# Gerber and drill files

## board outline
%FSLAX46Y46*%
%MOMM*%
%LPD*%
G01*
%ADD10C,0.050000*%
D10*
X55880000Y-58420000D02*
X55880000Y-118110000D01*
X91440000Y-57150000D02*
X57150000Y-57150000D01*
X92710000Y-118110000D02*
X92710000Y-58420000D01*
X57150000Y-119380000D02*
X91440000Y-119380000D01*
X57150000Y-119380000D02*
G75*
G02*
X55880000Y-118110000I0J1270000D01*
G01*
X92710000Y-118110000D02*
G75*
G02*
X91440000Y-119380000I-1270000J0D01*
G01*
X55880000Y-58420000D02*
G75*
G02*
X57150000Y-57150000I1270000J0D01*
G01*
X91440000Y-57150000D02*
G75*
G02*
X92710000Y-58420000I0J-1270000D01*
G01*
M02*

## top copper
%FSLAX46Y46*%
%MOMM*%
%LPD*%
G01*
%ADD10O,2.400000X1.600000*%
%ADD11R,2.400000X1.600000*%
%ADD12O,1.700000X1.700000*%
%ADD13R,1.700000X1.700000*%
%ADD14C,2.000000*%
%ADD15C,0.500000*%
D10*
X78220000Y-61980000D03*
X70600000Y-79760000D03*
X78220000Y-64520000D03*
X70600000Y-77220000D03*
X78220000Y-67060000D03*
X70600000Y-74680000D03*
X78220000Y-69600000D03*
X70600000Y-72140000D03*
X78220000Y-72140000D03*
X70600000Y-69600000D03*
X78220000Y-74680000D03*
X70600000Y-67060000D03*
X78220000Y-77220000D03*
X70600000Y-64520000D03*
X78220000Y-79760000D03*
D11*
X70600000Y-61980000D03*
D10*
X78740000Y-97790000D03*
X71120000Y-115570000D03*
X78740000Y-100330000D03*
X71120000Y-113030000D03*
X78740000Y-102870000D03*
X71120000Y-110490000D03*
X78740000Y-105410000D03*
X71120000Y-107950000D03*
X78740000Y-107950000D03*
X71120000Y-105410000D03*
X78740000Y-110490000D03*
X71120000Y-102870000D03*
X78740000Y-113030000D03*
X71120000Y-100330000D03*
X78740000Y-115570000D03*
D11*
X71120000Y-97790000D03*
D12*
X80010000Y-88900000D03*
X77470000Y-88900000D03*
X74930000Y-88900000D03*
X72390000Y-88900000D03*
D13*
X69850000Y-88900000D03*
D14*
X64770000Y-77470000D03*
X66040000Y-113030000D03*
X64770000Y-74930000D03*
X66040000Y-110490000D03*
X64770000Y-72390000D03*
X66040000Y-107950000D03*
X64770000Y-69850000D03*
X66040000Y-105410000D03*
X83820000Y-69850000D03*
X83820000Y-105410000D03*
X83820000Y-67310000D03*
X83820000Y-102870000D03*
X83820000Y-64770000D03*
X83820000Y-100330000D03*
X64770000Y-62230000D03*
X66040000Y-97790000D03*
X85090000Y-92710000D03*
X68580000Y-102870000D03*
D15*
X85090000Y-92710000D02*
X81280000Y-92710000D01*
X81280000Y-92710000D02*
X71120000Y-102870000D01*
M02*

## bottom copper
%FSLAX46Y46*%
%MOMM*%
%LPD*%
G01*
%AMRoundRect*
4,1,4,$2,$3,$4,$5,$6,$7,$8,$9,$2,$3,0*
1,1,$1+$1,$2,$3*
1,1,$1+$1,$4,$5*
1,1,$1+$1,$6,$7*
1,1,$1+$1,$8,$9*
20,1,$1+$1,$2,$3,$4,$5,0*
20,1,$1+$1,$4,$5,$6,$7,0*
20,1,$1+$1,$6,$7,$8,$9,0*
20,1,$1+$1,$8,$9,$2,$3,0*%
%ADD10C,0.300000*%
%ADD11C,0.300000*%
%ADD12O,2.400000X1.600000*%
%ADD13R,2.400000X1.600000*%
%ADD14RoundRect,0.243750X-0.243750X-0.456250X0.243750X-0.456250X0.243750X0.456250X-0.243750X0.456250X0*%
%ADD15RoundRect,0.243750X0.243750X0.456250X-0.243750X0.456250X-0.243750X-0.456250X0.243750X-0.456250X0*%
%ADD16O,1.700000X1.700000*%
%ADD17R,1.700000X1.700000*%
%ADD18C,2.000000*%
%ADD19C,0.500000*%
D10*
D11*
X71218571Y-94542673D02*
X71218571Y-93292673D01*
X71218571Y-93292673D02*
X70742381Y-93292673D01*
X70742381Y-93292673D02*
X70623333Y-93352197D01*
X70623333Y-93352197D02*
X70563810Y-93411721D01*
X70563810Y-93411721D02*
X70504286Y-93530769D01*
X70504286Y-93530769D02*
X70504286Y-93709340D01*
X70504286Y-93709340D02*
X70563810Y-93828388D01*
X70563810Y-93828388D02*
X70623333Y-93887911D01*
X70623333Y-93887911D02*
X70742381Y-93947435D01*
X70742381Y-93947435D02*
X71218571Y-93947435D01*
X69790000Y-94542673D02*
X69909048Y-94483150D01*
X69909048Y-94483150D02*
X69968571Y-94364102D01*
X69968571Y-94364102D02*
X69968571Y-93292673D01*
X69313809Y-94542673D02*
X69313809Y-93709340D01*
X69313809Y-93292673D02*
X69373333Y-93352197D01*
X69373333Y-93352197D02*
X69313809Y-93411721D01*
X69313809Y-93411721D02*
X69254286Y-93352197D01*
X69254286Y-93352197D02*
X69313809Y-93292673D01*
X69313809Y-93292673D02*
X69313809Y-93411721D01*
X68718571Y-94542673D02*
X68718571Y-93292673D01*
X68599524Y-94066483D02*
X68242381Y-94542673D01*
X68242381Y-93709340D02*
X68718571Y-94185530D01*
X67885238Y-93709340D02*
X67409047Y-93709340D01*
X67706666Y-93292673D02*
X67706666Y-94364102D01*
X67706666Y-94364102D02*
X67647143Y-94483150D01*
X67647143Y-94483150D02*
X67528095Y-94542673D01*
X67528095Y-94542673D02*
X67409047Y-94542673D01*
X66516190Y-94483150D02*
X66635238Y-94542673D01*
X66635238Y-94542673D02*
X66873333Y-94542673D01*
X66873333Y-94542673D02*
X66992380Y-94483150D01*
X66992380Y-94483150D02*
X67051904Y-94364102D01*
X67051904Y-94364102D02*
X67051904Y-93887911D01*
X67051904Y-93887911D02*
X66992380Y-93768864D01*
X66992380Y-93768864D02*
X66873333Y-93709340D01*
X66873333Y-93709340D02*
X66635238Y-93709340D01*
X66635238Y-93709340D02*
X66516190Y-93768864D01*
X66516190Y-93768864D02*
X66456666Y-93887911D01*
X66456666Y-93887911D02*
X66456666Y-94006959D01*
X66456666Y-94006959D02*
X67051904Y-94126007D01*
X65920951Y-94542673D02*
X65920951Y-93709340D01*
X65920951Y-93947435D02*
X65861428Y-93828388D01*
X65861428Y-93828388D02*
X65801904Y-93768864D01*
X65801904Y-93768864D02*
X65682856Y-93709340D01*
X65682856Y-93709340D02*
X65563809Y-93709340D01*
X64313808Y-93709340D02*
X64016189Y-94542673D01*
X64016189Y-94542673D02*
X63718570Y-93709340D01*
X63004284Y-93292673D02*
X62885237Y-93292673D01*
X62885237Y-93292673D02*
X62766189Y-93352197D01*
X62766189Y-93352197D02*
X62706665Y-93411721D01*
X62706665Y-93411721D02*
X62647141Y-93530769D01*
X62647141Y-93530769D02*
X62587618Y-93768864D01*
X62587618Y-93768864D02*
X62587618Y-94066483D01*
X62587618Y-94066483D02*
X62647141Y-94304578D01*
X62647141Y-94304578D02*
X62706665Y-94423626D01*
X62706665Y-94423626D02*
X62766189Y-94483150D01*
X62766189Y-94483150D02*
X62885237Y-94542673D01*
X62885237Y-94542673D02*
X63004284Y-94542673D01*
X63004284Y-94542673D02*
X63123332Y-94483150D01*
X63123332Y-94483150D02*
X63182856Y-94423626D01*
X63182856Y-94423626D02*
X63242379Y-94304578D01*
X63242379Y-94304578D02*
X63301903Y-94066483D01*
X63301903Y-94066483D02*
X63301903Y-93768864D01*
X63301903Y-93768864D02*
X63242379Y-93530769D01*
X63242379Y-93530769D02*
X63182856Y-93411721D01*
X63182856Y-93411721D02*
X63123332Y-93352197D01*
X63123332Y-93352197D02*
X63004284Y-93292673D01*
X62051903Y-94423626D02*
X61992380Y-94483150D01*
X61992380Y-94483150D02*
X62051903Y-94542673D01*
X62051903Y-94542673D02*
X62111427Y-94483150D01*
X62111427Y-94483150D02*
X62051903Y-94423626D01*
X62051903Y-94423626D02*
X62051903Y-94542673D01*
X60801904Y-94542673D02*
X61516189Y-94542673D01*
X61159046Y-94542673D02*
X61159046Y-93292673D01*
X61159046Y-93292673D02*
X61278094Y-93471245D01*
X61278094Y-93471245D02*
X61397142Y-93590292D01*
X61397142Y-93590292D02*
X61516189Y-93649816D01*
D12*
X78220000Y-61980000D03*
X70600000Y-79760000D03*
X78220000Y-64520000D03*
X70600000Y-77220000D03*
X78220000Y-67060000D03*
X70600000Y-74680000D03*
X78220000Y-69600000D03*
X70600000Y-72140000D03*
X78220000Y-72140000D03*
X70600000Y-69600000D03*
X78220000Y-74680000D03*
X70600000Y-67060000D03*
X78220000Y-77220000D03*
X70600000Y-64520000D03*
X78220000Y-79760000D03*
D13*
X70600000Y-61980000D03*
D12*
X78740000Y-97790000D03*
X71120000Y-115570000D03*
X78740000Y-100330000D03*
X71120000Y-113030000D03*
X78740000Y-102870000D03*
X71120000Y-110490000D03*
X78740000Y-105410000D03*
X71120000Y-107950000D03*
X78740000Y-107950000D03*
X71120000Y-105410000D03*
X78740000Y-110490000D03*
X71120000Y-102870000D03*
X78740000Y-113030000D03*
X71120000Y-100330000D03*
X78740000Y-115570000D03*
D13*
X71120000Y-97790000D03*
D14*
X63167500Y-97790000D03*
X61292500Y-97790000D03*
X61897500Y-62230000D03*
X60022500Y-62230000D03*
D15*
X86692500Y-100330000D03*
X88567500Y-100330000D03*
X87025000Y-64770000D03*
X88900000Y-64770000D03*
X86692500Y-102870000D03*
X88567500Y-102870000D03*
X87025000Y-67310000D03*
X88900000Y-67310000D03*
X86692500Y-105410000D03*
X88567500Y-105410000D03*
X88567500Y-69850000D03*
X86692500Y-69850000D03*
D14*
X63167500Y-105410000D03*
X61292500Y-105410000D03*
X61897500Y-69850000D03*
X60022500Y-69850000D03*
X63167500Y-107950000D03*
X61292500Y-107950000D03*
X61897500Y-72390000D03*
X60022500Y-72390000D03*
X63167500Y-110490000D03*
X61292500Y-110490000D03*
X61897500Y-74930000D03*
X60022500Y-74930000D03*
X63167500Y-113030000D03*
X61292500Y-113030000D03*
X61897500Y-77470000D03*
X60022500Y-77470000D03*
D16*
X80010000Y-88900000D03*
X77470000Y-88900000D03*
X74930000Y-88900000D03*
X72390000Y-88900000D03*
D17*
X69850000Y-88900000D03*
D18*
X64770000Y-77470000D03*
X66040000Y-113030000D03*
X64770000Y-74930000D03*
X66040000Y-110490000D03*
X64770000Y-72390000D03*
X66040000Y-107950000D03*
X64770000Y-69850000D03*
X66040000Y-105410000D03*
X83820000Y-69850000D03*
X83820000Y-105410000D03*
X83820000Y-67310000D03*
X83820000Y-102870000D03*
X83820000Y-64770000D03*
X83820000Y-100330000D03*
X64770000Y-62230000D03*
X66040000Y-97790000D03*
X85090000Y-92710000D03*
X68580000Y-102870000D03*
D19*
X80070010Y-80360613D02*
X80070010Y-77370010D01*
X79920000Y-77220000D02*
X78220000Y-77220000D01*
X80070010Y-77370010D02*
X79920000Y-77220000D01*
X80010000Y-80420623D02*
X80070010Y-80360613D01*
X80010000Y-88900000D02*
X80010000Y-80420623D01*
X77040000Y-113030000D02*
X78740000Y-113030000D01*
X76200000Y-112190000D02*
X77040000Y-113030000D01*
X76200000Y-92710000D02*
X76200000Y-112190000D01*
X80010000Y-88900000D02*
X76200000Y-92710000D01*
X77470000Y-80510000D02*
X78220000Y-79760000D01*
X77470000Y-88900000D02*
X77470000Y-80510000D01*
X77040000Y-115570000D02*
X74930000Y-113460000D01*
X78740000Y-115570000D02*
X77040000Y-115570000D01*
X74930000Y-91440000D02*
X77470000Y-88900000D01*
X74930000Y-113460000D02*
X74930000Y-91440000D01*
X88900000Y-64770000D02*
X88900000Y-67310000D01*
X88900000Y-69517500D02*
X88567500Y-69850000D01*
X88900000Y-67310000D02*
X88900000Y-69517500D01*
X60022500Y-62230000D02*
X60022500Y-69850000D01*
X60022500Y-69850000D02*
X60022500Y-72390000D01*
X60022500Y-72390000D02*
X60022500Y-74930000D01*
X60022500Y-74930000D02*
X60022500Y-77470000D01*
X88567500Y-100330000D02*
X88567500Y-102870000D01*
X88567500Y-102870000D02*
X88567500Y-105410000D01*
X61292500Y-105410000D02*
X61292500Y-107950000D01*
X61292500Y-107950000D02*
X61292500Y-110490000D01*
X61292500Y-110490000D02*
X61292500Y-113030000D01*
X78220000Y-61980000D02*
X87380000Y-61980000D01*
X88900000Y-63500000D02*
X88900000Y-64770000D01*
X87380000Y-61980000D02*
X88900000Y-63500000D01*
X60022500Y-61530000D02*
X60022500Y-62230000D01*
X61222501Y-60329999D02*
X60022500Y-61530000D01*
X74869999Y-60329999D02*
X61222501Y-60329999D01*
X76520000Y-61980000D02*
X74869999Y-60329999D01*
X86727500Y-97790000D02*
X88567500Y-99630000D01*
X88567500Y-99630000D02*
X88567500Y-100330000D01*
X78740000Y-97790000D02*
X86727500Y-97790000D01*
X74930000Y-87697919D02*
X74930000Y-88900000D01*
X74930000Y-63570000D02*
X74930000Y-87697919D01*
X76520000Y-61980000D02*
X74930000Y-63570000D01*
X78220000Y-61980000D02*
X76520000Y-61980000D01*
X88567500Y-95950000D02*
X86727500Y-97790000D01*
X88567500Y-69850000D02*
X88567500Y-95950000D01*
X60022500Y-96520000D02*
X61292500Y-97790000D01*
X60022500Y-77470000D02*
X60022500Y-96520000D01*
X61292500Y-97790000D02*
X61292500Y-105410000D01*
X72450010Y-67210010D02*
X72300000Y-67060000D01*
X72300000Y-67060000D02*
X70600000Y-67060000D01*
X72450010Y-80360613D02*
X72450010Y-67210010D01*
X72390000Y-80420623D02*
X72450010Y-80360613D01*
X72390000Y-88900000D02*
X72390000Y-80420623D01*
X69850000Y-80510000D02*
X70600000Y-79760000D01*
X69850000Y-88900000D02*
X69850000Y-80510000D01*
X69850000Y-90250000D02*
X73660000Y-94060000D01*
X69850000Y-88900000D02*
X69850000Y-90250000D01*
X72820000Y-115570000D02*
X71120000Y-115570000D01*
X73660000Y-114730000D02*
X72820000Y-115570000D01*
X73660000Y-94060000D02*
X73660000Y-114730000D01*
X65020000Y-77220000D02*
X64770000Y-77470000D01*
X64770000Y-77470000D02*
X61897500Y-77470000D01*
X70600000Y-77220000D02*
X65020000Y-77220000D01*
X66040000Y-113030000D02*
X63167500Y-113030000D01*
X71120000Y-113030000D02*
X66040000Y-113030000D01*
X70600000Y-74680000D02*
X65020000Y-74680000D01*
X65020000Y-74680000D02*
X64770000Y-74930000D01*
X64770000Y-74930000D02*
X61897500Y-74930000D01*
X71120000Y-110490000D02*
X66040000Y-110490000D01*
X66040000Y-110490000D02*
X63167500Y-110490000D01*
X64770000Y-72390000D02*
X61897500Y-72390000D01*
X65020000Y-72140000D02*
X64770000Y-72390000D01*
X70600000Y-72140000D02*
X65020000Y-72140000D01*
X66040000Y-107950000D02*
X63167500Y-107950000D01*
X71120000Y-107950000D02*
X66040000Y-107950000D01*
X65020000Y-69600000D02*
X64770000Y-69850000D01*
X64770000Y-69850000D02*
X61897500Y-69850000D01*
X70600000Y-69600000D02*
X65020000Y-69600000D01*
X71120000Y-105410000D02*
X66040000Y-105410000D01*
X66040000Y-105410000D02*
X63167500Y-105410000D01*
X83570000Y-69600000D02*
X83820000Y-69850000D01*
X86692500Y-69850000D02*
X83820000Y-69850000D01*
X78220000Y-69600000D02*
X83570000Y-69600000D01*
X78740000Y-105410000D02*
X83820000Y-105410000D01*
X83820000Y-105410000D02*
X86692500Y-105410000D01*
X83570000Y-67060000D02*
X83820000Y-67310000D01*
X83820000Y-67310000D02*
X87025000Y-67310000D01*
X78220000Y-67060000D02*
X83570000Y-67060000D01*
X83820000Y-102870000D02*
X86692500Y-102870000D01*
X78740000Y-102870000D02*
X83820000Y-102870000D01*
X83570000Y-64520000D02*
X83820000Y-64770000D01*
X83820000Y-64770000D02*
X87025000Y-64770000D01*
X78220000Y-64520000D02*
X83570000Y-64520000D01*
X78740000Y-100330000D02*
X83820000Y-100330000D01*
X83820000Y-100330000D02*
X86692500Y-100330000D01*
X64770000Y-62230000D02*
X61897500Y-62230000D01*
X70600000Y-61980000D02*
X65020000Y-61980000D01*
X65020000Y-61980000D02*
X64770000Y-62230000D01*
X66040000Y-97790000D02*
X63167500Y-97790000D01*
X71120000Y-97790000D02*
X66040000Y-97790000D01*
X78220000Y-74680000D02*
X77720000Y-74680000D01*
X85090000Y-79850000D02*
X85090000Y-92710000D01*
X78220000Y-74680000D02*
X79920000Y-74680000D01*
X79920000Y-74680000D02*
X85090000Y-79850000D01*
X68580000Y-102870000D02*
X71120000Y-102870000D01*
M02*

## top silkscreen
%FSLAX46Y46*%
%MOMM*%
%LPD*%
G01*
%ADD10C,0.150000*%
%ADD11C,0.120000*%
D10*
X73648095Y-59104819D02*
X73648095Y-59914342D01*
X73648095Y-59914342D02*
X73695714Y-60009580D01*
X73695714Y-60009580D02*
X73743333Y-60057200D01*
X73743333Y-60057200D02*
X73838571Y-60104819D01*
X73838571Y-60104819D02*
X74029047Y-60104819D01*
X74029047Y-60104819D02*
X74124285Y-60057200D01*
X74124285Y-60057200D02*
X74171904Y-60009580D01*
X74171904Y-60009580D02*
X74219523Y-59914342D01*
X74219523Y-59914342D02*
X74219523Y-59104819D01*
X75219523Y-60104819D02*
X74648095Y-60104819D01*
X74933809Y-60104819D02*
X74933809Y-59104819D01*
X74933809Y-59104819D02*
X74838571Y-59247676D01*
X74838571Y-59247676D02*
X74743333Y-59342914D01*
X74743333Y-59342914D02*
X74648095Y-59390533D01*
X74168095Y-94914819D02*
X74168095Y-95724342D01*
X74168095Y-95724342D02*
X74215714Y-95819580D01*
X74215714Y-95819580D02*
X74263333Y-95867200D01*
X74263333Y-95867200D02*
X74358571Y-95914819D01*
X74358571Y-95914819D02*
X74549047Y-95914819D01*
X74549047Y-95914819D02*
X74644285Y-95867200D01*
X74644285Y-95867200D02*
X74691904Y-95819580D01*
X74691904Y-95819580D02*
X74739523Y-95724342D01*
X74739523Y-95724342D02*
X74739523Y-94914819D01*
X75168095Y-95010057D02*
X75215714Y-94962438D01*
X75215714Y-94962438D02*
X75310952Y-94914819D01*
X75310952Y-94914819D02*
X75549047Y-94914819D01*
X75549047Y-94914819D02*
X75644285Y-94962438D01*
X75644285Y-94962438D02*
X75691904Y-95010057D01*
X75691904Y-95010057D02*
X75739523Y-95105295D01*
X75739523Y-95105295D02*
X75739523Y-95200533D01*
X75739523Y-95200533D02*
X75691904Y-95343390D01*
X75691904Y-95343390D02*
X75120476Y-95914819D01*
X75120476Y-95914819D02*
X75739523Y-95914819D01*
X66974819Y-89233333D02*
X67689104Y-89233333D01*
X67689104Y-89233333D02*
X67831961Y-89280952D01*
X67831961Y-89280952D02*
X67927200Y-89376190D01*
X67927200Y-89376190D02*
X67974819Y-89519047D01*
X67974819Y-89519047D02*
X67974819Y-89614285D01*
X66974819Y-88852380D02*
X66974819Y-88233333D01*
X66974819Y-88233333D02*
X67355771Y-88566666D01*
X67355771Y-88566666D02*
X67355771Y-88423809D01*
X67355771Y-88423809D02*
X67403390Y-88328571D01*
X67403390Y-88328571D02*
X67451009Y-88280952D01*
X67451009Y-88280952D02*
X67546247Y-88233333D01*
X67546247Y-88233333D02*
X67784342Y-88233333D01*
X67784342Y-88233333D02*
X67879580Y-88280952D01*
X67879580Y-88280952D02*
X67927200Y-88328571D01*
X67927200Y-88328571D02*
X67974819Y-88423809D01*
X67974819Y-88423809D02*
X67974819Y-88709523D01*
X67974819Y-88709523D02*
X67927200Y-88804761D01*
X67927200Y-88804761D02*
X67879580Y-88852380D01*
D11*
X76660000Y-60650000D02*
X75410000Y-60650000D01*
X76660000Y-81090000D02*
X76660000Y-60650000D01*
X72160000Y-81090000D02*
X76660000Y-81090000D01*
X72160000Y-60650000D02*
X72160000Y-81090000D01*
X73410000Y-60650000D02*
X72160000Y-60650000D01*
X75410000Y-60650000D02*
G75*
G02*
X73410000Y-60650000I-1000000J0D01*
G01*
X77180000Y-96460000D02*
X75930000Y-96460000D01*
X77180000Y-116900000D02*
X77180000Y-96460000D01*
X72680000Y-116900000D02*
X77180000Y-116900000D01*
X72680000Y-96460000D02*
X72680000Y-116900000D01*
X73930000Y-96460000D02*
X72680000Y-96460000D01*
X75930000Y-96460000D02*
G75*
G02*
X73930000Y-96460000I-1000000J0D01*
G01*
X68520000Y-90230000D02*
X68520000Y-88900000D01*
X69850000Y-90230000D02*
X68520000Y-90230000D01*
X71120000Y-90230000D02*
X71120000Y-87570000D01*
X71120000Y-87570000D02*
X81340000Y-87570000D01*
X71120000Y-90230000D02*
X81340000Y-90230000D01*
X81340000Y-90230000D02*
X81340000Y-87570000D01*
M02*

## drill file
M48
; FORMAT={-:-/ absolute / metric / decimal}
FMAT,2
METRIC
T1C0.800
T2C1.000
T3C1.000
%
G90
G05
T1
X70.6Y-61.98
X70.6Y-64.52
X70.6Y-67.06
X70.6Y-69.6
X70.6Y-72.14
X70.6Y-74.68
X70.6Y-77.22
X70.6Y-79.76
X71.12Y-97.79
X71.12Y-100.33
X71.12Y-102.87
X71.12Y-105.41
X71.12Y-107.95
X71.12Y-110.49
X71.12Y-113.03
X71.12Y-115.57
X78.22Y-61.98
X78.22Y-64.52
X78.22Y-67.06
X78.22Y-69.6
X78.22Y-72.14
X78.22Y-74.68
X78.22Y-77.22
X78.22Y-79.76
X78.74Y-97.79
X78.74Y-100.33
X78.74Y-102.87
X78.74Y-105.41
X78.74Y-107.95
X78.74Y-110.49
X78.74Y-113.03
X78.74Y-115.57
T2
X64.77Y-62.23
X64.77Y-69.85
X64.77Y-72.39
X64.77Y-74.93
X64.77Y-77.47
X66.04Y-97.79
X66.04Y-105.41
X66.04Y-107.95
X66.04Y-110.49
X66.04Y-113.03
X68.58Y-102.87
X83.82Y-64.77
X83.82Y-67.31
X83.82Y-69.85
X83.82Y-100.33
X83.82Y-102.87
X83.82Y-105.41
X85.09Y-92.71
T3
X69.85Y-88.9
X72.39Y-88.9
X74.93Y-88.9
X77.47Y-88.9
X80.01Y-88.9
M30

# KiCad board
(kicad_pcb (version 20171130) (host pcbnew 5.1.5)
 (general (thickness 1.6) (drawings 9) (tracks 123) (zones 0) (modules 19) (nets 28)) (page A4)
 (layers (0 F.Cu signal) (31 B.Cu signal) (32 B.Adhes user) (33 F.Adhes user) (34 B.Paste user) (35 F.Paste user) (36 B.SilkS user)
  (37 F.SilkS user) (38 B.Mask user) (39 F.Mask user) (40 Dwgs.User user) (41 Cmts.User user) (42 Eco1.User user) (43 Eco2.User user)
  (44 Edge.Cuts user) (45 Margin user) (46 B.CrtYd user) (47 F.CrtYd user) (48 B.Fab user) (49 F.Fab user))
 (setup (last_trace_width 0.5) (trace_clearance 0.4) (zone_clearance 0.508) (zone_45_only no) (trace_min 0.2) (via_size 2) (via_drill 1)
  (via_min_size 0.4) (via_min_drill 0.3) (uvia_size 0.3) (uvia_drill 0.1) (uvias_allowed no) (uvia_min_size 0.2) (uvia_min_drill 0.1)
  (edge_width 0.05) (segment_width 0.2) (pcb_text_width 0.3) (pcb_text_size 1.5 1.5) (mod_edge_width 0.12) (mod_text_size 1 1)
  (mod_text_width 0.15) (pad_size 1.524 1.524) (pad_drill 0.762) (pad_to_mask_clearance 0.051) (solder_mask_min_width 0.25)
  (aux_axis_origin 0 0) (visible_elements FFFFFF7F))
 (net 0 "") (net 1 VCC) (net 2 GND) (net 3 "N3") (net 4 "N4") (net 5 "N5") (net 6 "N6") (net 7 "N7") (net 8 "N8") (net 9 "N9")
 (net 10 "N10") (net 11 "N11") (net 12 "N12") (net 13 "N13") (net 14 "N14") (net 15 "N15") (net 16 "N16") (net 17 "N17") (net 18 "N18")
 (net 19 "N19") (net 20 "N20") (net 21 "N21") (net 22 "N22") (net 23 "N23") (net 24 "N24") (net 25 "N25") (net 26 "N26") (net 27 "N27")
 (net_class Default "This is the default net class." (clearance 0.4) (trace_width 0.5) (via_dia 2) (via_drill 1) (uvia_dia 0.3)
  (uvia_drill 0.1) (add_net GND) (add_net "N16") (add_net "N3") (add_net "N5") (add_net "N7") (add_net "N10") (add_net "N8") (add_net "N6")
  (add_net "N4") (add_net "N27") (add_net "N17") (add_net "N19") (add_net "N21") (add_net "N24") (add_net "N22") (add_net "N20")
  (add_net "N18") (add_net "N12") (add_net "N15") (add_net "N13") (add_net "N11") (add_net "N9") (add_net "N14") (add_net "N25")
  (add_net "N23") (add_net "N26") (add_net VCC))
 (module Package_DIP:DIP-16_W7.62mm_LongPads (layer F.Cu) (at 70.6 61.98)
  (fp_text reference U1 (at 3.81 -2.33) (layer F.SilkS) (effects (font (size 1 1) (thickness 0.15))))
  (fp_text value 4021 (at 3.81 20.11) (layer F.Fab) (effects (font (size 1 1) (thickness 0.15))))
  (fp_line (start 6.06 -1.33) (end 4.81 -1.33) (layer F.SilkS) (width 0.12))
  (fp_line (start 6.06 19.11) (end 6.06 -1.33) (layer F.SilkS) (width 0.12))
  (fp_line (start 1.56 19.11) (end 6.06 19.11) (layer F.SilkS) (width 0.12))
  (fp_line (start 1.56 -1.33) (end 1.56 19.11) (layer F.SilkS) (width 0.12))
  (fp_line (start 2.81 -1.33) (end 1.56 -1.33) (layer F.SilkS) (width 0.12))
  (fp_arc (start 3.81 -1.33) (end 2.81 -1.33) (angle -180) (layer F.SilkS) (width 0.12))
  (pad 16 thru_hole oval (at 7.62 0) (size 2.4 1.6) (drill 0.8) (layers *.Cu *.Mask) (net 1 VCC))
  (pad 8 thru_hole oval (at 0 17.78) (size 2.4 1.6) (drill 0.8) (layers *.Cu *.Mask) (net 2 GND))
  (pad 15 thru_hole oval (at 7.62 2.54) (size 2.4 1.6) (drill 0.8) (layers *.Cu *.Mask) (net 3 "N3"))
  (pad 7 thru_hole oval (at 0 15.24) (size 2.4 1.6) (drill 0.8) (layers *.Cu *.Mask) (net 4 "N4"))
  (pad 14 thru_hole oval (at 7.62 5.08) (size 2.4 1.6) (drill 0.8) (layers *.Cu *.Mask) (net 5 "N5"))
  (pad 6 thru_hole oval (at 0 12.7) (size 2.4 1.6) (drill 0.8) (layers *.Cu *.Mask) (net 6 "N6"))
  (pad 13 thru_hole oval (at 7.62 7.62) (size 2.4 1.6) (drill 0.8) (layers *.Cu *.Mask) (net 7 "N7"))
  (pad 5 thru_hole oval (at 0 10.16) (size 2.4 1.6) (drill 0.8) (layers *.Cu *.Mask) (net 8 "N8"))
  (pad 12 thru_hole oval (at 7.62 10.16) (size 2.4 1.6) (drill 0.8) (layers *.Cu *.Mask) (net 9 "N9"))
  (pad 4 thru_hole oval (at 0 7.62) (size 2.4 1.6) (drill 0.8) (layers *.Cu *.Mask) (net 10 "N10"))
  (pad 11 thru_hole oval (at 7.62 12.7) (size 2.4 1.6) (drill 0.8) (layers *.Cu *.Mask) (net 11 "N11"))
  (pad 3 thru_hole oval (at 0 5.08) (size 2.4 1.6) (drill 0.8) (layers *.Cu *.Mask) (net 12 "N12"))
  (pad 10 thru_hole oval (at 7.62 15.24) (size 2.4 1.6) (drill 0.8) (layers *.Cu *.Mask) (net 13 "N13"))
  (pad 2 thru_hole oval (at 0 2.54) (size 2.4 1.6) (drill 0.8) (layers *.Cu *.Mask) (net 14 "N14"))
  (pad 9 thru_hole oval (at 7.62 17.78) (size 2.4 1.6) (drill 0.8) (layers *.Cu *.Mask) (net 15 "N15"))
  (pad 1 thru_hole rect (at 0 0) (size 2.4 1.6) (drill 0.8) (layers *.Cu *.Mask) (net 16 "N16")))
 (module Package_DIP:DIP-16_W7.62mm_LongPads (layer F.Cu) (at 71.12 97.79)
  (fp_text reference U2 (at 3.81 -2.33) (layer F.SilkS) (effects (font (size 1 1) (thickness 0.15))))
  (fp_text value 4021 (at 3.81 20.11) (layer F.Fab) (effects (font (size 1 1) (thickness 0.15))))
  (fp_line (start 6.06 -1.33) (end 4.81 -1.33) (layer F.SilkS) (width 0.12))
  (fp_line (start 6.06 19.11) (end 6.06 -1.33) (layer F.SilkS) (width 0.12))
  (fp_line (start 1.56 19.11) (end 6.06 19.11) (layer F.SilkS) (width 0.12))
  (fp_line (start 1.56 -1.33) (end 1.56 19.11) (layer F.SilkS) (width 0.12))
  (fp_line (start 2.81 -1.33) (end 1.56 -1.33) (layer F.SilkS) (width 0.12))
  (fp_arc (start 3.81 -1.33) (end 2.81 -1.33) (angle -180) (layer F.SilkS) (width 0.12))
  (pad 16 thru_hole oval (at 7.62 0) (size 2.4 1.6) (drill 0.8) (layers *.Cu *.Mask) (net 1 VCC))
  (pad 8 thru_hole oval (at 0 17.78) (size 2.4 1.6) (drill 0.8) (layers *.Cu *.Mask) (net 2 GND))
  (pad 15 thru_hole oval (at 7.62 2.54) (size 2.4 1.6) (drill 0.8) (layers *.Cu *.Mask) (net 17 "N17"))
  (pad 7 thru_hole oval (at 0 15.24) (size 2.4 1.6) (drill 0.8) (layers *.Cu *.Mask) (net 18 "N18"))
  (pad 14 thru_hole oval (at 7.62 5.08) (size 2.4 1.6) (drill 0.8) (layers *.Cu *.Mask) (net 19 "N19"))
  (pad 6 thru_hole oval (at 0 12.7) (size 2.4 1.6) (drill 0.8) (layers *.Cu *.Mask) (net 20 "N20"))
  (pad 13 thru_hole oval (at 7.62 7.62) (size 2.4 1.6) (drill 0.8) (layers *.Cu *.Mask) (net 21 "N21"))
  (pad 5 thru_hole oval (at 0 10.16) (size 2.4 1.6) (drill 0.8) (layers *.Cu *.Mask) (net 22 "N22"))
  (pad 12 thru_hole oval (at 7.62 10.16) (size 2.4 1.6) (drill 0.8) (layers *.Cu *.Mask) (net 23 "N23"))
  (pad 4 thru_hole oval (at 0 7.62) (size 2.4 1.6) (drill 0.8) (layers *.Cu *.Mask) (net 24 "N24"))
  (pad 11 thru_hole oval (at 7.62 12.7) (size 2.4 1.6) (drill 0.8) (layers *.Cu *.Mask) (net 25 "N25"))
  (pad 3 thru_hole oval (at 0 5.08) (size 2.4 1.6) (drill 0.8) (layers *.Cu *.Mask) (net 11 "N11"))
  (pad 10 thru_hole oval (at 7.62 15.24) (size 2.4 1.6) (drill 0.8) (layers *.Cu *.Mask) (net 13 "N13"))
  (pad 2 thru_hole oval (at 0 2.54) (size 2.4 1.6) (drill 0.8) (layers *.Cu *.Mask) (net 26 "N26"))
  (pad 9 thru_hole oval (at 7.62 17.78) (size 2.4 1.6) (drill 0.8) (layers *.Cu *.Mask) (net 15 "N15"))
  (pad 1 thru_hole rect (at 0 0) (size 2.4 1.6) (drill 0.8) (layers *.Cu *.Mask) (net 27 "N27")))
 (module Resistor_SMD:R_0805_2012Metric (layer B.Cu) (at 62.23 97.79)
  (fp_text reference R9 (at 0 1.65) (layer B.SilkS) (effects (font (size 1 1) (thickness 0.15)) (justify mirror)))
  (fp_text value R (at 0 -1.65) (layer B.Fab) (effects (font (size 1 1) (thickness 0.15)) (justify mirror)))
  (pad 2 smd roundrect (at 0.9375 0) (size 0.975 1.4) (layers B.Cu B.Paste B.Mask) (roundrect_rratio 0.25) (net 27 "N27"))
  (pad 1 smd roundrect (at -0.9375 0) (size 0.975 1.4) (layers B.Cu B.Paste B.Mask) (roundrect_rratio 0.25) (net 1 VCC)))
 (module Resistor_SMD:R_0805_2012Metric (layer B.Cu) (at 60.96 62.23)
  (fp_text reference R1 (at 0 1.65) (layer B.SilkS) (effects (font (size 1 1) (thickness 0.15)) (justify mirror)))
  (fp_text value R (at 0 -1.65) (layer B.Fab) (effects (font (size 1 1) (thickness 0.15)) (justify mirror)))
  (pad 2 smd roundrect (at 0.9375 0) (size 0.975 1.4) (layers B.Cu B.Paste B.Mask) (roundrect_rratio 0.25) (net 16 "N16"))
  (pad 1 smd roundrect (at -0.9375 0) (size 0.975 1.4) (layers B.Cu B.Paste B.Mask) (roundrect_rratio 0.25) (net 1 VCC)))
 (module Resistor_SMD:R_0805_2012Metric (layer B.Cu) (at 87.63 100.33 180)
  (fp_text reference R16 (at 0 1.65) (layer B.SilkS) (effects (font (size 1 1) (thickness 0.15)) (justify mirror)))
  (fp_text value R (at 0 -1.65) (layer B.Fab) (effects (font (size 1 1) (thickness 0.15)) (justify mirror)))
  (pad 2 smd roundrect (at 0.9375 0 180) (size 0.975 1.4) (layers B.Cu B.Paste B.Mask) (roundrect_rratio 0.25) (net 17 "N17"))
  (pad 1 smd roundrect (at -0.9375 0 180) (size 0.975 1.4) (layers B.Cu B.Paste B.Mask) (roundrect_rratio 0.25) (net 1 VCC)))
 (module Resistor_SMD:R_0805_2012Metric (layer B.Cu) (at 87.9625 64.77 180)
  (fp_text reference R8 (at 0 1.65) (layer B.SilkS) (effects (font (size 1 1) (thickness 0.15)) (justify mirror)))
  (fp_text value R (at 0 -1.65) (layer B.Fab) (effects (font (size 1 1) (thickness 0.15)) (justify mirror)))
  (pad 2 smd roundrect (at 0.9375 0 180) (size 0.975 1.4) (layers B.Cu B.Paste B.Mask) (roundrect_rratio 0.25) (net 3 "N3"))
  (pad 1 smd roundrect (at -0.9375 0 180) (size 0.975 1.4) (layers B.Cu B.Paste B.Mask) (roundrect_rratio 0.25) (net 1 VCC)))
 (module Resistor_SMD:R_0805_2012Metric (layer B.Cu) (at 87.63 102.87 180)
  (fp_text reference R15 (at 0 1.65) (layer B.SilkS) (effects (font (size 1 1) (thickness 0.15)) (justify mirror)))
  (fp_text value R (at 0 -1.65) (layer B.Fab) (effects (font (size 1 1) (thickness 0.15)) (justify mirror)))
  (pad 2 smd roundrect (at 0.9375 0 180) (size 0.975 1.4) (layers B.Cu B.Paste B.Mask) (roundrect_rratio 0.25) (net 19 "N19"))
  (pad 1 smd roundrect (at -0.9375 0 180) (size 0.975 1.4) (layers B.Cu B.Paste B.Mask) (roundrect_rratio 0.25) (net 1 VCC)))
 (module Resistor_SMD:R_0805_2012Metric (layer B.Cu) (at 87.9625 67.31 180)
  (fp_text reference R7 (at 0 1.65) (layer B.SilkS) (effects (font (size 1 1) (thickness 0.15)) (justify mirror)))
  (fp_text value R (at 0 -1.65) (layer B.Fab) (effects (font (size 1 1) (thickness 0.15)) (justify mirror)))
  (pad 2 smd roundrect (at 0.9375 0 180) (size 0.975 1.4) (layers B.Cu B.Paste B.Mask) (roundrect_rratio 0.25) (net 5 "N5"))
  (pad 1 smd roundrect (at -0.9375 0 180) (size 0.975 1.4) (layers B.Cu B.Paste B.Mask) (roundrect_rratio 0.25) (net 1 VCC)))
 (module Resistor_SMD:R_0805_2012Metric (layer B.Cu) (at 87.63 105.41 180)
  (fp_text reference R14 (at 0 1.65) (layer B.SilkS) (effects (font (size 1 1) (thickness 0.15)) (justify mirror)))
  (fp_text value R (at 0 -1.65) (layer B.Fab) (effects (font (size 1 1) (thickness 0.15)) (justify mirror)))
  (pad 2 smd roundrect (at 0.9375 0 180) (size 0.975 1.4) (layers B.Cu B.Paste B.Mask) (roundrect_rratio 0.25) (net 21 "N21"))
  (pad 1 smd roundrect (at -0.9375 0 180) (size 0.975 1.4) (layers B.Cu B.Paste B.Mask) (roundrect_rratio 0.25) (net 1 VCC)))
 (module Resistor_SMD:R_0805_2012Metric (layer B.Cu) (at 87.63 69.85 180)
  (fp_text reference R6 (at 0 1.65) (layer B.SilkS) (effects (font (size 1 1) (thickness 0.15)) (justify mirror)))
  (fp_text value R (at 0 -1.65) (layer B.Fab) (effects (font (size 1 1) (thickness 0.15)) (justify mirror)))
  (pad 1 smd roundrect (at -0.9375 0 180) (size 0.975 1.4) (layers B.Cu B.Paste B.Mask) (roundrect_rratio 0.25) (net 1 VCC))
  (pad 2 smd roundrect (at 0.9375 0 180) (size 0.975 1.4) (layers B.Cu B.Paste B.Mask) (roundrect_rratio 0.25) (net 7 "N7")))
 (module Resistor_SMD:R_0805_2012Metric (layer B.Cu) (at 62.23 105.41)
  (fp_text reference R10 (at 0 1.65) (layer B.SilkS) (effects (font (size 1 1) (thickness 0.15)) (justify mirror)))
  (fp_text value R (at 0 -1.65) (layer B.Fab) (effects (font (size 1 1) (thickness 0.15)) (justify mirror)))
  (pad 2 smd roundrect (at 0.9375 0) (size 0.975 1.4) (layers B.Cu B.Paste B.Mask) (roundrect_rratio 0.25) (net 24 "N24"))
  (pad 1 smd roundrect (at -0.9375 0) (size 0.975 1.4) (layers B.Cu B.Paste B.Mask) (roundrect_rratio 0.25) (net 1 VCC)))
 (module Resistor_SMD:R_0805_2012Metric (layer B.Cu) (at 60.96 69.85)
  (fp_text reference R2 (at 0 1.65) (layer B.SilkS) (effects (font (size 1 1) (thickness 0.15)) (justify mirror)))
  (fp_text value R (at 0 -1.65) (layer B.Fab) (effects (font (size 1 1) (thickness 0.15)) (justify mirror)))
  (pad 2 smd roundrect (at 0.9375 0) (size 0.975 1.4) (layers B.Cu B.Paste B.Mask) (roundrect_rratio 0.25) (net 10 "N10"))
  (pad 1 smd roundrect (at -0.9375 0) (size 0.975 1.4) (layers B.Cu B.Paste B.Mask) (roundrect_rratio 0.25) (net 1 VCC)))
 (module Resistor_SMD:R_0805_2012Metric (layer B.Cu) (at 62.23 107.95)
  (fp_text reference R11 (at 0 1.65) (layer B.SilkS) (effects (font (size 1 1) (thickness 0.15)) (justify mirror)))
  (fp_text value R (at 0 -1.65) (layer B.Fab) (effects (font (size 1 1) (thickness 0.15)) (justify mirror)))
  (pad 2 smd roundrect (at 0.9375 0) (size 0.975 1.4) (layers B.Cu B.Paste B.Mask) (roundrect_rratio 0.25) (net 22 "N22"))
  (pad 1 smd roundrect (at -0.9375 0) (size 0.975 1.4) (layers B.Cu B.Paste B.Mask) (roundrect_rratio 0.25) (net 1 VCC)))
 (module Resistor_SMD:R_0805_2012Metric (layer B.Cu) (at 60.96 72.39)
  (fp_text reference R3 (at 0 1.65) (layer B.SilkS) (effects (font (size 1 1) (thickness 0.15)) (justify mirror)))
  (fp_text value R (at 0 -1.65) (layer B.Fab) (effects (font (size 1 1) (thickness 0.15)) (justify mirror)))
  (pad 2 smd roundrect (at 0.9375 0) (size 0.975 1.4) (layers B.Cu B.Paste B.Mask) (roundrect_rratio 0.25) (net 8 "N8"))
  (pad 1 smd roundrect (at -0.9375 0) (size 0.975 1.4) (layers B.Cu B.Paste B.Mask) (roundrect_rratio 0.25) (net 1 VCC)))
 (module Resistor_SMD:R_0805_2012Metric (layer B.Cu) (at 62.23 110.49)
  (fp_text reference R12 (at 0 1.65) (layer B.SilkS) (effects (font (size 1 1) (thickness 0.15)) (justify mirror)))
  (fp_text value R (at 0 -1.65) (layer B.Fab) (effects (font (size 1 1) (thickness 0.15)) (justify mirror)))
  (pad 2 smd roundrect (at 0.9375 0) (size 0.975 1.4) (layers B.Cu B.Paste B.Mask) (roundrect_rratio 0.25) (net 20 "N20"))
  (pad 1 smd roundrect (at -0.9375 0) (size 0.975 1.4) (layers B.Cu B.Paste B.Mask) (roundrect_rratio 0.25) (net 1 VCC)))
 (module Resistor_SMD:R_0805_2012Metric (layer B.Cu) (at 60.96 74.93)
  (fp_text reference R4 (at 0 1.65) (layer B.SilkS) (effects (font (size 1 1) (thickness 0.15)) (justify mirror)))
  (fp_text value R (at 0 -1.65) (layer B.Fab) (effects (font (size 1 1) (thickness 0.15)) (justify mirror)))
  (pad 2 smd roundrect (at 0.9375 0) (size 0.975 1.4) (layers B.Cu B.Paste B.Mask) (roundrect_rratio 0.25) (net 6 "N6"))
  (pad 1 smd roundrect (at -0.9375 0) (size 0.975 1.4) (layers B.Cu B.Paste B.Mask) (roundrect_rratio 0.25) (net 1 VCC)))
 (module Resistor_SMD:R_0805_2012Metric (layer B.Cu) (at 62.23 113.03)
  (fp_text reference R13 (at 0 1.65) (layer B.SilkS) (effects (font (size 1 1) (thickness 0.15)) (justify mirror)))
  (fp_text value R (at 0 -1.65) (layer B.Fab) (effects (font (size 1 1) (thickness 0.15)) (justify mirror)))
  (pad 2 smd roundrect (at 0.9375 0) (size 0.975 1.4) (layers B.Cu B.Paste B.Mask) (roundrect_rratio 0.25) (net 18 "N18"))
  (pad 1 smd roundrect (at -0.9375 0) (size 0.975 1.4) (layers B.Cu B.Paste B.Mask) (roundrect_rratio 0.25) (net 1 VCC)))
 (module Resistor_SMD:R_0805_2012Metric (layer B.Cu) (at 60.96 77.47)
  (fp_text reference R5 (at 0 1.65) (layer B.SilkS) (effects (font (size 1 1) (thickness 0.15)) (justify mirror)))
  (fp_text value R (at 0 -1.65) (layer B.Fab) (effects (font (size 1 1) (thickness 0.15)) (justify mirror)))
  (pad 2 smd roundrect (at 0.9375 0) (size 0.975 1.4) (layers B.Cu B.Paste B.Mask) (roundrect_rratio 0.25) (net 4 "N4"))
  (pad 1 smd roundrect (at -0.9375 0) (size 0.975 1.4) (layers B.Cu B.Paste B.Mask) (roundrect_rratio 0.25) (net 1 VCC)))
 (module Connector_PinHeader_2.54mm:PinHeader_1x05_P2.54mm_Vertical (layer F.Cu) (at 69.85 88.9 90)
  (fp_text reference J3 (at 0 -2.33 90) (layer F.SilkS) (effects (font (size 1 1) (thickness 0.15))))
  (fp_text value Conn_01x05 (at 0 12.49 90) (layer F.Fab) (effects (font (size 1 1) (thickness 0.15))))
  (fp_line (start -1.33 -1.33) (end 0 -1.33) (layer F.SilkS) (width 0.12))
  (fp_line (start -1.33 0) (end -1.33 -1.33) (layer F.SilkS) (width 0.12))
  (fp_line (start -1.33 1.27) (end 1.33 1.27) (layer F.SilkS) (width 0.12))
  (fp_line (start 1.33 1.27) (end 1.33 11.49) (layer F.SilkS) (width 0.12))
  (fp_line (start -1.33 1.27) (end -1.33 11.49) (layer F.SilkS) (width 0.12))
  (fp_line (start -1.33 11.49) (end 1.33 11.49) (layer F.SilkS) (width 0.12))
  (pad 5 thru_hole oval (at 0 10.16 90) (size 1.7 1.7) (drill 1) (layers *.Cu *.Mask) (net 13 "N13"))
  (pad 4 thru_hole oval (at 0 7.62 90) (size 1.7 1.7) (drill 1) (layers *.Cu *.Mask) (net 15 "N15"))
  (pad 3 thru_hole oval (at 0 5.08 90) (size 1.7 1.7) (drill 1) (layers *.Cu *.Mask) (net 1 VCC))
  (pad 2 thru_hole oval (at 0 2.54 90) (size 1.7 1.7) (drill 1) (layers *.Cu *.Mask) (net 12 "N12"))
  (pad 1 thru_hole rect (at 0 0 90) (size 1.7 1.7) (drill 1) (layers *.Cu *.Mask) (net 2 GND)))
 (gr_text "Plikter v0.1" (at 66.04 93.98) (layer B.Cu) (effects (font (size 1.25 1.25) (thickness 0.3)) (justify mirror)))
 (gr_line (start 55.88 58.42) (end 55.88 118.11) (layer Edge.Cuts) (width 0.05))
 (gr_line (start 91.44 57.15) (end 57.15 57.15) (layer Edge.Cuts) (width 0.05))
 (gr_line (start 92.71 118.11) (end 92.71 58.42) (layer Edge.Cuts) (width 0.05))
 (gr_line (start 57.15 119.38) (end 91.44 119.38) (layer Edge.Cuts) (width 0.05))
 (gr_arc (start 57.15 118.11) (end 55.88 118.11) (angle -90) (layer Edge.Cuts) (width 0.05))
 (gr_arc (start 91.44 118.11) (end 91.44 119.38) (angle -90) (layer Edge.Cuts) (width 0.05))
 (gr_arc (start 57.15 58.42) (end 57.15 57.15) (angle -90) (layer Edge.Cuts) (width 0.05))
 (gr_arc (start 91.44 58.42) (end 92.71 58.42) (angle -90) (layer Edge.Cuts) (width 0.05))
 (segment (start 80.07001 80.360613) (end 80.07001 77.37001) (width 0.5) (layer B.Cu) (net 13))
 (segment (start 79.92 77.22) (end 78.22 77.22) (width 0.5) (layer B.Cu) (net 13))
 (segment (start 80.07001 77.37001) (end 79.92 77.22) (width 0.5) (layer B.Cu) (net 13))
 (segment (start 80.01 80.420623) (end 80.07001 80.360613) (width 0.5) (layer B.Cu) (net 13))
 (segment (start 80.01 88.9) (end 80.01 80.420623) (width 0.5) (layer B.Cu) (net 13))
 (segment (start 77.04 113.03) (end 78.74 113.03) (width 0.5) (layer B.Cu) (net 13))
 (segment (start 76.2 112.19) (end 77.04 113.03) (width 0.5) (layer B.Cu) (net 13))
 (segment (start 76.2 92.71) (end 76.2 112.19) (width 0.5) (layer B.Cu) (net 13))
 (segment (start 80.01 88.9) (end 76.2 92.71) (width 0.5) (layer B.Cu) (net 13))
 (segment (start 77.47 80.51) (end 78.22 79.76) (width 0.5) (layer B.Cu) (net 15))
 (segment (start 77.47 88.9) (end 77.47 80.51) (width 0.5) (layer B.Cu) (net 15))
 (segment (start 77.04 115.57) (end 74.93 113.46) (width 0.5) (layer B.Cu) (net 15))
 (segment (start 78.74 115.57) (end 77.04 115.57) (width 0.5) (layer B.Cu) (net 15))
 (segment (start 74.93 91.44) (end 77.47 88.9) (width 0.5) (layer B.Cu) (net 15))
 (segment (start 74.93 113.46) (end 74.93 91.44) (width 0.5) (layer B.Cu) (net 15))
 (segment (start 88.9 64.77) (end 88.9 67.31) (width 0.5) (layer B.Cu) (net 1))
 (segment (start 88.9 69.5175) (end 88.5675 69.85) (width 0.5) (layer B.Cu) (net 1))
 (segment (start 88.9 67.31) (end 88.9 69.5175) (width 0.5) (layer B.Cu) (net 1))
 (segment (start 60.0225 62.23) (end 60.0225 69.85) (width 0.5) (layer B.Cu) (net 1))
 (segment (start 60.0225 69.85) (end 60.0225 72.39) (width 0.5) (layer B.Cu) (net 1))
 (segment (start 60.0225 72.39) (end 60.0225 74.93) (width 0.5) (layer B.Cu) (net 1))
 (segment (start 60.0225 74.93) (end 60.0225 77.47) (width 0.5) (layer B.Cu) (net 1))
 (segment (start 88.5675 100.33) (end 88.5675 102.87) (width 0.5) (layer B.Cu) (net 1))
 (segment (start 88.5675 102.87) (end 88.5675 105.41) (width 0.5) (layer B.Cu) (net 1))
 (segment (start 61.2925 105.41) (end 61.2925 107.95) (width 0.5) (layer B.Cu) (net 1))
 (segment (start 61.2925 107.95) (end 61.2925 110.49) (width 0.5) (layer B.Cu) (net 1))
 (segment (start 61.2925 110.49) (end 61.2925 113.03) (width 0.5) (layer B.Cu) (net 1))
 (segment (start 78.22 61.98) (end 87.38 61.98) (width 0.5) (layer B.Cu) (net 1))
 (segment (start 88.9 63.5) (end 88.9 64.77) (width 0.5) (layer B.Cu) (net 1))
 (segment (start 87.38 61.98) (end 88.9 63.5) (width 0.5) (layer B.Cu) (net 1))
 (segment (start 60.0225 61.53) (end 60.0225 62.23) (width 0.5) (layer B.Cu) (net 1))
 (segment (start 61.222501 60.329999) (end 60.0225 61.53) (width 0.5) (layer B.Cu) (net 1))
 (segment (start 74.869999 60.329999) (end 61.222501 60.329999) (width 0.5) (layer B.Cu) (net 1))
 (segment (start 76.52 61.98) (end 74.869999 60.329999) (width 0.5) (layer B.Cu) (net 1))
 (segment (start 86.7275 97.79) (end 88.5675 99.63) (width 0.5) (layer B.Cu) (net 1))
 (segment (start 88.5675 99.63) (end 88.5675 100.33) (width 0.5) (layer B.Cu) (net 1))
 (segment (start 78.74 97.79) (end 86.7275 97.79) (width 0.5) (layer B.Cu) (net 1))
 (segment (start 74.93 87.697919) (end 74.93 88.9) (width 0.5) (layer B.Cu) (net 1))
 (segment (start 74.93 63.57) (end 74.93 87.697919) (width 0.5) (layer B.Cu) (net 1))
 (segment (start 76.52 61.98) (end 74.93 63.57) (width 0.5) (layer B.Cu) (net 1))
 (segment (start 78.22 61.98) (end 76.52 61.98) (width 0.5) (layer B.Cu) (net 1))
 (segment (start 88.5675 95.95) (end 86.7275 97.79) (width 0.5) (layer B.Cu) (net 1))
 (segment (start 88.5675 69.85) (end 88.5675 95.95) (width 0.5) (layer B.Cu) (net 1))
 (segment (start 60.0225 96.52) (end 61.2925 97.79) (width 0.5) (layer B.Cu) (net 1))
 (segment (start 60.0225 77.47) (end 60.0225 96.52) (width 0.5) (layer B.Cu) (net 1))
 (segment (start 61.2925 97.79) (end 61.2925 105.41) (width 0.5) (layer B.Cu) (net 1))
 (segment (start 72.45001 67.21001) (end 72.3 67.06) (width 0.5) (layer B.Cu) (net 12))
 (segment (start 72.3 67.06) (end 70.6 67.06) (width 0.5) (layer B.Cu) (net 12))
 (segment (start 72.45001 80.360613) (end 72.45001 67.21001) (width 0.5) (layer B.Cu) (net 12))
 (segment (start 72.39 80.420623) (end 72.45001 80.360613) (width 0.5) (layer B.Cu) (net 12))
 (segment (start 72.39 88.9) (end 72.39 80.420623) (width 0.5) (layer B.Cu) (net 12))
 (segment (start 69.85 80.51) (end 70.6 79.76) (width 0.5) (layer B.Cu) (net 2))
 (segment (start 69.85 88.9) (end 69.85 80.51) (width 0.5) (layer B.Cu) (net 2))
 (segment (start 69.85 90.25) (end 73.66 94.06) (width 0.5) (layer B.Cu) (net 2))
 (segment (start 69.85 88.9) (end 69.85 90.25) (width 0.5) (layer B.Cu) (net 2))
 (segment (start 72.82 115.57) (end 71.12 115.57) (width 0.5) (layer B.Cu) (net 2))
 (segment (start 73.66 114.73) (end 72.82 115.57) (width 0.5) (layer B.Cu) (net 2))
 (segment (start 73.66 94.06) (end 73.66 114.73) (width 0.5) (layer B.Cu) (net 2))
 (segment (start 65.02 77.22) (end 64.77 77.47) (width 0.5) (layer B.Cu) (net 4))
 (via (at 64.77 77.47) (size 2) (drill 1) (layers F.Cu B.Cu) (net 4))
 (segment (start 64.77 77.47) (end 61.8975 77.47) (width 0.5) (layer B.Cu) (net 4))
 (segment (start 70.6 77.22) (end 65.02 77.22) (width 0.5) (layer B.Cu) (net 4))
 (segment (start 66.04 113.03) (end 63.1675 113.03) (width 0.5) (layer B.Cu) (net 18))
 (via (at 66.04 113.03) (size 2) (drill 1) (layers F.Cu B.Cu) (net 18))
 (segment (start 71.12 113.03) (end 66.04 113.03) (width 0.5) (layer B.Cu) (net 18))
 (segment (start 70.6 74.68) (end 65.02 74.68) (width 0.5) (layer B.Cu) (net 6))
 (segment (start 65.02 74.68) (end 64.77 74.93) (width 0.5) (layer B.Cu) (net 6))
 (segment (start 64.77 74.93) (end 61.8975 74.93) (width 0.5) (layer B.Cu) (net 6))
 (via (at 64.77 74.93) (size 2) (drill 1) (layers F.Cu B.Cu) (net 6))
 (segment (start 71.12 110.49) (end 66.04 110.49) (width 0.5) (layer B.Cu) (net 20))
 (via (at 66.04 110.49) (size 2) (drill 1) (layers F.Cu B.Cu) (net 20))
 (segment (start 66.04 110.49) (end 63.1675 110.49) (width 0.5) (layer B.Cu) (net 20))
 (segment (start 64.77 72.39) (end 61.8975 72.39) (width 0.5) (layer B.Cu) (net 8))
 (via (at 64.77 72.39) (size 2) (drill 1) (layers F.Cu B.Cu) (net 8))
 (segment (start 65.02 72.14) (end 64.77 72.39) (width 0.5) (layer B.Cu) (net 8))
 (segment (start 70.6 72.14) (end 65.02 72.14) (width 0.5) (layer B.Cu) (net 8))
 (segment (start 66.04 107.95) (end 63.1675 107.95) (width 0.5) (layer B.Cu) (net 22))
 (via (at 66.04 107.95) (size 2) (drill 1) (layers F.Cu B.Cu) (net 22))
 (segment (start 71.12 107.95) (end 66.04 107.95) (width 0.5) (layer B.Cu) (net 22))
 (segment (start 65.02 69.6) (end 64.77 69.85) (width 0.5) (layer B.Cu) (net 10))
 (segment (start 64.77 69.85) (end 61.8975 69.85) (width 0.5) (layer B.Cu) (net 10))
 (segment (start 70.6 69.6) (end 65.02 69.6) (width 0.5) (layer B.Cu) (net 10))
 (via (at 64.77 69.85) (size 2) (drill 1) (layers F.Cu B.Cu) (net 10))
 (segment (start 71.12 105.41) (end 66.04 105.41) (width 0.5) (layer B.Cu) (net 24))
 (via (at 66.04 105.41) (size 2) (drill 1) (layers F.Cu B.Cu) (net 24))
 (segment (start 66.04 105.41) (end 63.1675 105.41) (width 0.5) (layer B.Cu) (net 24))
 (segment (start 83.57 69.6) (end 83.82 69.85) (width 0.5) (layer B.Cu) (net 7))
 (via (at 83.82 69.85) (size 2) (drill 1) (layers F.Cu B.Cu) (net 7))
 (segment (start 86.6925 69.85) (end 83.82 69.85) (width 0.5) (layer B.Cu) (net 7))
 (segment (start 78.22 69.6) (end 83.57 69.6) (width 0.5) (layer B.Cu) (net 7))
 (via (at 83.82 105.41) (size 2) (drill 1) (layers F.Cu B.Cu) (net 21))
 (segment (start 78.74 105.41) (end 83.82 105.41) (width 0.5) (layer B.Cu) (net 21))
 (segment (start 83.82 105.41) (end 86.6925 105.41) (width 0.5) (layer B.Cu) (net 21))
 (via (at 83.82 67.31) (size 2) (drill 1) (layers F.Cu B.Cu) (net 5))
 (segment (start 83.57 67.06) (end 83.82 67.31) (width 0.5) (layer B.Cu) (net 5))
 (segment (start 83.82 67.31) (end 87.025 67.31) (width 0.5) (layer B.Cu) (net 5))
 (segment (start 78.22 67.06) (end 83.57 67.06) (width 0.5) (layer B.Cu) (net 5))
 (segment (start 83.82 102.87) (end 86.6925 102.87) (width 0.5) (layer B.Cu) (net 19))
 (via (at 83.82 102.87) (size 2) (drill 1) (layers F.Cu B.Cu) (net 19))
 (segment (start 78.74 102.87) (end 83.82 102.87) (width 0.5) (layer B.Cu) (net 19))
 (via (at 83.82 64.77) (size 2) (drill 1) (layers F.Cu B.Cu) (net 3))
 (segment (start 83.57 64.52) (end 83.82 64.77) (width 0.5) (layer B.Cu) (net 3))
 (segment (start 83.82 64.77) (end 87.025 64.77) (width 0.5) (layer B.Cu) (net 3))
 (segment (start 78.22 64.52) (end 83.57 64.52) (width 0.5) (layer B.Cu) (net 3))
 (via (at 83.82 100.33) (size 2) (drill 1) (layers F.Cu B.Cu) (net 17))
 (segment (start 78.74 100.33) (end 83.82 100.33) (width 0.5) (layer B.Cu) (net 17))
 (segment (start 83.82 100.33) (end 86.6925 100.33) (width 0.5) (layer B.Cu) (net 17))
 (segment (start 64.77 62.23) (end 61.8975 62.23) (width 0.5) (layer B.Cu) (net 16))
 (segment (start 70.6 61.98) (end 65.02 61.98) (width 0.5) (layer B.Cu) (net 16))
 (segment (start 65.02 61.98) (end 64.77 62.23) (width 0.5) (layer B.Cu) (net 16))
 (via (at 64.77 62.23) (size 2) (drill 1) (layers F.Cu B.Cu) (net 16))
 (segment (start 66.04 97.79) (end 63.1675 97.79) (width 0.5) (layer B.Cu) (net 27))
 (segment (start 71.12 97.79) (end 66.04 97.79) (width 0.5) (layer B.Cu) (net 27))
 (via (at 66.04 97.79) (size 2) (drill 1) (layers F.Cu B.Cu) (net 27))
 (segment (start 78.22 74.68) (end 77.72 74.68) (width 0.5) (layer B.Cu) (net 11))
 (segment (start 85.09 79.85) (end 85.09 92.71) (width 0.5) (layer B.Cu) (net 11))
 (via (at 85.09 92.71) (size 2) (drill 1) (layers F.Cu B.Cu) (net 11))
 (segment (start 78.22 74.68) (end 79.92 74.68) (width 0.5) (layer B.Cu) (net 11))
 (segment (start 79.92 74.68) (end 85.09 79.85) (width 0.5) (layer B.Cu) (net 11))
 (via (at 68.58 102.87) (size 2) (drill 1) (layers F.Cu B.Cu) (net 11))
 (segment (start 85.09 92.71) (end 81.28 92.71) (width 0.5) (layer F.Cu) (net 11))
 (segment (start 81.28 92.71) (end 71.12 102.87) (width 0.5) (layer F.Cu) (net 11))
 (segment (start 68.58 102.87) (end 71.12 102.87) (width 0.5) (layer B.Cu) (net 11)))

